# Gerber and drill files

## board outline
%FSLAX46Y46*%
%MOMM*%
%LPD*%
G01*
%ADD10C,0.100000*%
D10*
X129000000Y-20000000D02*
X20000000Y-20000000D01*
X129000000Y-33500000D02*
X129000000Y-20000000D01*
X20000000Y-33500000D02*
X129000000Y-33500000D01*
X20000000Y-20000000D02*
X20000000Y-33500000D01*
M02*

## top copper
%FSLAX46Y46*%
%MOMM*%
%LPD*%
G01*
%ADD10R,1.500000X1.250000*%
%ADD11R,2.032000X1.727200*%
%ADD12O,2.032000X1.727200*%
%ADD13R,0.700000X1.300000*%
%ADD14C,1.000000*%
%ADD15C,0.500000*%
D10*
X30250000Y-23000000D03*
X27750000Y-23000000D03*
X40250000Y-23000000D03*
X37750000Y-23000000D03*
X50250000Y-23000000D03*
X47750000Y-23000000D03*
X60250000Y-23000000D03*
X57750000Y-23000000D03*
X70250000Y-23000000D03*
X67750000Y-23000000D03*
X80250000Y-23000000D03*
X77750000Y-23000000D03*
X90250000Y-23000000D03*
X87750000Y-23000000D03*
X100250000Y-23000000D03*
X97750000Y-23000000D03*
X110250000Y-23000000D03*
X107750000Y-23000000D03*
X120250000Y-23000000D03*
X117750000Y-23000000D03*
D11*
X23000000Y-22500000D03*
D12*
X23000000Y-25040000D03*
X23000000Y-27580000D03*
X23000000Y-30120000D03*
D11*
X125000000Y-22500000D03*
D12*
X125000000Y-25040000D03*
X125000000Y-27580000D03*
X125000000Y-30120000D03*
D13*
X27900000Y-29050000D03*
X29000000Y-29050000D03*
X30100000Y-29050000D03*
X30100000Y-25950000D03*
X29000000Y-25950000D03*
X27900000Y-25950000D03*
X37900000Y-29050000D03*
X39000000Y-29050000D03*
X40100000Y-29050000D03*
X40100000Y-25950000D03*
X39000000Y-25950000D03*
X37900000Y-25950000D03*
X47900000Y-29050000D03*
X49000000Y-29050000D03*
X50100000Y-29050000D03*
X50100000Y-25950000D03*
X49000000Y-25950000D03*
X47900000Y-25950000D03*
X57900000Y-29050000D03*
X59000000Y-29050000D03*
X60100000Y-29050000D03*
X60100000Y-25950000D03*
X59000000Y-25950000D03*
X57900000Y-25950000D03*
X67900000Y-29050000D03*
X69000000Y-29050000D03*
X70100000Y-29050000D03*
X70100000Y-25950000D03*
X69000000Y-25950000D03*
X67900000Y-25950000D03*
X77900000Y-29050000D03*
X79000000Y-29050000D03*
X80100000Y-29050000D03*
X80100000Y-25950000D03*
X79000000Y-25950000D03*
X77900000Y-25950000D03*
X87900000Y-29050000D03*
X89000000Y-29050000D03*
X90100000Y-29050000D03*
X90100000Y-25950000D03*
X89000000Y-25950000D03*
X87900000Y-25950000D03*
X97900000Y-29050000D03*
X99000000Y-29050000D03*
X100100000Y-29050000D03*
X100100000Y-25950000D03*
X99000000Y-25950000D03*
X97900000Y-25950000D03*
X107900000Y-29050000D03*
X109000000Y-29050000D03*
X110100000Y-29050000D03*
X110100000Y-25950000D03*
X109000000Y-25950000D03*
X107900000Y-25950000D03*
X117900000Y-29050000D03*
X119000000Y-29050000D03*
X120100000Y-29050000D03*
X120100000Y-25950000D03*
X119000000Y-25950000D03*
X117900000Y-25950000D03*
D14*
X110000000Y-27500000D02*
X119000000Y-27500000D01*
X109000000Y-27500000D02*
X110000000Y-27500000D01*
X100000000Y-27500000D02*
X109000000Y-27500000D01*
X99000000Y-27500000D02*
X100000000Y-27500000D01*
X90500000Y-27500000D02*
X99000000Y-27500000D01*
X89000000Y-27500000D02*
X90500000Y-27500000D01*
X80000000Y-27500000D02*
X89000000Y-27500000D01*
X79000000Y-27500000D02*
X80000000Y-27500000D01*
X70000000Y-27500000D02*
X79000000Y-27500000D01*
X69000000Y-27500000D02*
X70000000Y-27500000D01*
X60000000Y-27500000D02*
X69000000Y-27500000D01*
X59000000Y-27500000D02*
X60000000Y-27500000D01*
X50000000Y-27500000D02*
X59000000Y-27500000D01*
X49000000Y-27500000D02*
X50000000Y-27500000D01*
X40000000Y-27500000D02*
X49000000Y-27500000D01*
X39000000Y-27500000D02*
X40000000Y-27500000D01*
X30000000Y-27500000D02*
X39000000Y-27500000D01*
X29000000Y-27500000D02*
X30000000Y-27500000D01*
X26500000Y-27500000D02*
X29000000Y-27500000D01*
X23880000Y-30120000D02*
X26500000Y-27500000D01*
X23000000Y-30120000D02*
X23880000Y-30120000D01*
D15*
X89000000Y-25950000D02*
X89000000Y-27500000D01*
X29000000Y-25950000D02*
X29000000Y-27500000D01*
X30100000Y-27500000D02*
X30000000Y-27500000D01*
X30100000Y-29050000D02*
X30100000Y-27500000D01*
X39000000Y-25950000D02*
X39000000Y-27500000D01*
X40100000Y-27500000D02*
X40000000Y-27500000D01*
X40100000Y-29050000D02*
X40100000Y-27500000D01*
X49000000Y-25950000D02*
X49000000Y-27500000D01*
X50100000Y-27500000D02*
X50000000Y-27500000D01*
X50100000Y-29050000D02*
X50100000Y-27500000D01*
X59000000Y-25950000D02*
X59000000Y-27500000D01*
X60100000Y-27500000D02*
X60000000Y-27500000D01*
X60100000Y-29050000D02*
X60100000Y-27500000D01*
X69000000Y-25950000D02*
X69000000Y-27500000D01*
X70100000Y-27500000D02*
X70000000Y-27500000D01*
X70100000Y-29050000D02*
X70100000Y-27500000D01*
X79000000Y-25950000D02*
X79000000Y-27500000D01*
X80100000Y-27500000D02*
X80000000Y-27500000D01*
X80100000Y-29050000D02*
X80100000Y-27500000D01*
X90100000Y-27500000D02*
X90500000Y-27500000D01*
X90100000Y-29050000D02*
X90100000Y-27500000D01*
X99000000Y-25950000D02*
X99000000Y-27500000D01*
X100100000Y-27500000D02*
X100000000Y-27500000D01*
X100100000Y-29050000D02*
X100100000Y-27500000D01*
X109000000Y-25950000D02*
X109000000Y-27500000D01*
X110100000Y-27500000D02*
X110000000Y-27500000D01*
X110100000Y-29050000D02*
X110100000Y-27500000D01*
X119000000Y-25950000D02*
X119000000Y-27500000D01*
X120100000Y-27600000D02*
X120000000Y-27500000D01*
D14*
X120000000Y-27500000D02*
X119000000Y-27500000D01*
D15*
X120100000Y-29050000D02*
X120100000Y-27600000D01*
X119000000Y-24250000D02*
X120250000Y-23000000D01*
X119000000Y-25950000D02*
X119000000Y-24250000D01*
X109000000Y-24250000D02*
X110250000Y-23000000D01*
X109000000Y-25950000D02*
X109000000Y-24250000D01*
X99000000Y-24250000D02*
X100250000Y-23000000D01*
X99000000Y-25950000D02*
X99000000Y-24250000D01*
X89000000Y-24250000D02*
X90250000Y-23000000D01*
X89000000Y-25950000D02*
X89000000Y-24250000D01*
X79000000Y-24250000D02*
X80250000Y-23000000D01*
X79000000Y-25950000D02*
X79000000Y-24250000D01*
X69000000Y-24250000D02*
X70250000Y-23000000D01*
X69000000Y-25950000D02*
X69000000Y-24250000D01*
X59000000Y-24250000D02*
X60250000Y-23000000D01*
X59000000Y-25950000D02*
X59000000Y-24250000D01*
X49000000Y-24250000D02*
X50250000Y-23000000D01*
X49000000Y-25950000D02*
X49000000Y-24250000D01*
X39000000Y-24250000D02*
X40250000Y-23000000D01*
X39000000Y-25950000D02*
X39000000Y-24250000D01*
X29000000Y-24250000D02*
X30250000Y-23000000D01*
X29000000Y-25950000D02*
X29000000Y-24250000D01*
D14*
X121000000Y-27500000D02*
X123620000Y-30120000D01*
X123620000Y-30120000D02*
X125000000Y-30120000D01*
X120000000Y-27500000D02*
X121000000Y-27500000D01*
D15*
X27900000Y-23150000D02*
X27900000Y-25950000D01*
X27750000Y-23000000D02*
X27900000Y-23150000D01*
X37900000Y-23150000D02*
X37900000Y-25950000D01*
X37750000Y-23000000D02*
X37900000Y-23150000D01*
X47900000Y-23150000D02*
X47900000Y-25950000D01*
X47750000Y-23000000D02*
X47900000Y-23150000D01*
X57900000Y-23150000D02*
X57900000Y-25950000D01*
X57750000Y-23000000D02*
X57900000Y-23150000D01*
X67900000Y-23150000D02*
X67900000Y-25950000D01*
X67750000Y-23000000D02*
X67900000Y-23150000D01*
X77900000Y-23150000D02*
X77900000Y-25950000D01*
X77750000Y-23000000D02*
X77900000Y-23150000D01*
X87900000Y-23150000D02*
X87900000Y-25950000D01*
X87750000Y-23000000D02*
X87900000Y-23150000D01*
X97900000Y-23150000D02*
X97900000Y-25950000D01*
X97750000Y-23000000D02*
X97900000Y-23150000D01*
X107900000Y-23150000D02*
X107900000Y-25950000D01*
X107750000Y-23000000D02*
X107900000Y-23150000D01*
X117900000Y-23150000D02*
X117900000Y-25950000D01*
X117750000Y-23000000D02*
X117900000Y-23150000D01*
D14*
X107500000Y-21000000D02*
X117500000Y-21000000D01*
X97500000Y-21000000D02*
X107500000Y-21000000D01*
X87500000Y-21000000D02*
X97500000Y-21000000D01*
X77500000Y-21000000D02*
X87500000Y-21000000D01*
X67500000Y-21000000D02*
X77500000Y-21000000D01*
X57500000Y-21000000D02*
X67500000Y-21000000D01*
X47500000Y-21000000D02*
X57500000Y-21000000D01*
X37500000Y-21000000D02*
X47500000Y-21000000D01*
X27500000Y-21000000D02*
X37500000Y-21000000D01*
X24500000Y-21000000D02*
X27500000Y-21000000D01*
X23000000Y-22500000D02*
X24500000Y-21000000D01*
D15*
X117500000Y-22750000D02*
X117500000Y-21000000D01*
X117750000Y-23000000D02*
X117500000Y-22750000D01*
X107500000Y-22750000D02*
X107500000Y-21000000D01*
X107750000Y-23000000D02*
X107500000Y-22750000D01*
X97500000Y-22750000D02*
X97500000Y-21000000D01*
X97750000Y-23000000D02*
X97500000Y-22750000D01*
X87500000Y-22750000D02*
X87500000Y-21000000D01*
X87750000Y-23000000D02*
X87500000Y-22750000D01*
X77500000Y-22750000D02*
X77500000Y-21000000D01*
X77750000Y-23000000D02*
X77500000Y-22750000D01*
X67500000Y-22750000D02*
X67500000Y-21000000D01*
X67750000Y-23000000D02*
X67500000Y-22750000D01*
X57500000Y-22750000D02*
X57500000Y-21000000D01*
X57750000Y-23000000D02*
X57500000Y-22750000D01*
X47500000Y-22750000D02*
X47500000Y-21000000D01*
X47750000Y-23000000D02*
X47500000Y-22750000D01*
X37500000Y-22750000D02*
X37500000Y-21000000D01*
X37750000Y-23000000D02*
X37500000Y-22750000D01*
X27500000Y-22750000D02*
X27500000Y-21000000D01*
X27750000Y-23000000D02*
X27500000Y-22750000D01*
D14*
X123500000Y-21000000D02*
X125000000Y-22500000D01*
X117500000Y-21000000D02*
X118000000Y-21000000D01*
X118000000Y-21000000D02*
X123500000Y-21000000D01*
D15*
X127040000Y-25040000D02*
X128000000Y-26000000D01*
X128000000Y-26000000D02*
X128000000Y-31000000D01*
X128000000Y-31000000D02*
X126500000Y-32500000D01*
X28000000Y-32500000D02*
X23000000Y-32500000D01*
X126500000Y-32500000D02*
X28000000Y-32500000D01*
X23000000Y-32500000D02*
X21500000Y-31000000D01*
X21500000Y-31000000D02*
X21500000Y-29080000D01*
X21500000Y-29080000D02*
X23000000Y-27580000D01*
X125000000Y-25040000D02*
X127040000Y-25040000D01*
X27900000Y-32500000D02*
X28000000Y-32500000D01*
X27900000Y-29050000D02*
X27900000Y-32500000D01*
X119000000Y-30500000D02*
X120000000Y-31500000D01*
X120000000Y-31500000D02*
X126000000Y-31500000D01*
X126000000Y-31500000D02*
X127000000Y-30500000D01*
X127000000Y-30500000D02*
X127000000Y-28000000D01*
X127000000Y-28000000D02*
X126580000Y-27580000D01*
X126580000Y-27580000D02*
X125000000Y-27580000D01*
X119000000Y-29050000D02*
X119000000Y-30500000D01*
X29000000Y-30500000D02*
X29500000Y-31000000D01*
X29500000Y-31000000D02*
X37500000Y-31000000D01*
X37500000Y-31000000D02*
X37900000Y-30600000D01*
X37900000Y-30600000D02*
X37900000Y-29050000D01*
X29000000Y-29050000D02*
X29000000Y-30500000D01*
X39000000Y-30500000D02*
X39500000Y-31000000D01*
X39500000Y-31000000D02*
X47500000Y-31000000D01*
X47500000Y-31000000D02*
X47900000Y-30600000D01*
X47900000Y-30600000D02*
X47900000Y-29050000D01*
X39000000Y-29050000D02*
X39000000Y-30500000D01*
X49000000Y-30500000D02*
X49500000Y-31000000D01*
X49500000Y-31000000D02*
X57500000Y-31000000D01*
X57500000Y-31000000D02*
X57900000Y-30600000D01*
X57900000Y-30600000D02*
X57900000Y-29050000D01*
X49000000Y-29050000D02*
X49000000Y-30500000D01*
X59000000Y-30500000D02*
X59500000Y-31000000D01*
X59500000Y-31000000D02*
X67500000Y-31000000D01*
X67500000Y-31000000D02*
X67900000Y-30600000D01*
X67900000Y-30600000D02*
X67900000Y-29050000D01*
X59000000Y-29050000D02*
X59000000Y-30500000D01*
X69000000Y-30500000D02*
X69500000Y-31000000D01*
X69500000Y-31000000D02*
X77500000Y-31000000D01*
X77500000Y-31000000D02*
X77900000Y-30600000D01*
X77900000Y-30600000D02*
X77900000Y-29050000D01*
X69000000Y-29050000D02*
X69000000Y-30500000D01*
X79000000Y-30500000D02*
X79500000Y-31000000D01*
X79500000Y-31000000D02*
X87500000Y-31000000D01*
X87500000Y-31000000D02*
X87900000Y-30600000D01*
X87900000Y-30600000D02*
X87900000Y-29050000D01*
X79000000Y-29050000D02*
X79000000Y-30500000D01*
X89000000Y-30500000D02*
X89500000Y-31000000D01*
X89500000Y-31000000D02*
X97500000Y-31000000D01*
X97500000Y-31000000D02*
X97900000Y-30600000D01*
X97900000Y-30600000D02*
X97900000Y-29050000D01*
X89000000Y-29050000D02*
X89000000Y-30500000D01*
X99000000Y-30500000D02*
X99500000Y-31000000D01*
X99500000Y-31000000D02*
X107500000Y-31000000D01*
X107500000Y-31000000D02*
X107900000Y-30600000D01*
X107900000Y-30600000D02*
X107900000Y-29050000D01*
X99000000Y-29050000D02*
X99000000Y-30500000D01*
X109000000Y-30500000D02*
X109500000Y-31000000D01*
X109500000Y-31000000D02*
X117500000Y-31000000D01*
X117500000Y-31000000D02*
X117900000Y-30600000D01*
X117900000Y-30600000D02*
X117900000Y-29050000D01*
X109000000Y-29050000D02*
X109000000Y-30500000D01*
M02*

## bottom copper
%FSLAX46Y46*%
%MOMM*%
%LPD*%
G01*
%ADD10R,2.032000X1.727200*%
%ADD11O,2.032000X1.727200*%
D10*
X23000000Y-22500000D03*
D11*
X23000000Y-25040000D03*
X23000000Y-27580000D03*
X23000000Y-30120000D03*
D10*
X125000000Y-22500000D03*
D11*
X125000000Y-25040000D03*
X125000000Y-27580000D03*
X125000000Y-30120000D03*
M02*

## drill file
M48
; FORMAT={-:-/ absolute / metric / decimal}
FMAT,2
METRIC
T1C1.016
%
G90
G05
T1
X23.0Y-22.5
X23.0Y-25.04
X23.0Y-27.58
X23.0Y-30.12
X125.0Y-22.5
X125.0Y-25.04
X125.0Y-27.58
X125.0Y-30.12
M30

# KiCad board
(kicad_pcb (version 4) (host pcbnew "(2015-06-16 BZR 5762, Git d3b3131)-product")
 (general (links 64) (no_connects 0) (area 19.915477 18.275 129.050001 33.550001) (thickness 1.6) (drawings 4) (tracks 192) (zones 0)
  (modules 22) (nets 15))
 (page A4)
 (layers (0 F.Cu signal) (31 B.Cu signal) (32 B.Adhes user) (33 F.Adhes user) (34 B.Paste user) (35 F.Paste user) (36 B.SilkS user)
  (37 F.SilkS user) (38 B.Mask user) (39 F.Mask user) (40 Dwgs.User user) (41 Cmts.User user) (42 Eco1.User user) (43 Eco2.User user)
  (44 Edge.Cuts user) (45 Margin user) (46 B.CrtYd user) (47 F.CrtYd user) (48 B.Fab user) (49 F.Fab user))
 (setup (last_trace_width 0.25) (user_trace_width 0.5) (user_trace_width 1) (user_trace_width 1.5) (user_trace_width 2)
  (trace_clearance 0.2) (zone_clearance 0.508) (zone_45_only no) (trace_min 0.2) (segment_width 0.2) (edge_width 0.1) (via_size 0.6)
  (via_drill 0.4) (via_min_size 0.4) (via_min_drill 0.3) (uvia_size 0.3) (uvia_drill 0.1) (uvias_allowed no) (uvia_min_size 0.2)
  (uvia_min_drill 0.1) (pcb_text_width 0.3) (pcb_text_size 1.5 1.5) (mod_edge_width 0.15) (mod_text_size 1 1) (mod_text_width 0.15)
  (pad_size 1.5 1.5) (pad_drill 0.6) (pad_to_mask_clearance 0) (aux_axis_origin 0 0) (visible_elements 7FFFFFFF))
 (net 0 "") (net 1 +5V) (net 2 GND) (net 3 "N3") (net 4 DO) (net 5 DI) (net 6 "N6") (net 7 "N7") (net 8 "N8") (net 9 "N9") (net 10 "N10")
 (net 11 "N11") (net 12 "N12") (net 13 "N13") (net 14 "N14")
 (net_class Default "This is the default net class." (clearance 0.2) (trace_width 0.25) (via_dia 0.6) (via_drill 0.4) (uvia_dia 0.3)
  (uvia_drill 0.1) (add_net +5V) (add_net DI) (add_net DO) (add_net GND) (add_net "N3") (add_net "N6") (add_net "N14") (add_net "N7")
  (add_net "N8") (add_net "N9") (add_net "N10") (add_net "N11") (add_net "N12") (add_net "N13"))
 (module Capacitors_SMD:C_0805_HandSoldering (layer F.Cu) (at 29 23 180)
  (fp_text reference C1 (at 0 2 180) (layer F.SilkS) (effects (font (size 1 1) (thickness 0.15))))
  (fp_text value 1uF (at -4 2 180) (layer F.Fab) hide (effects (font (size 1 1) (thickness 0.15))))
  (pad 1 smd rect (at -1.25 0 180) (size 1.5 1.25) (layers F.Cu F.Paste F.Mask) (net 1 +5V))
  (pad 2 smd rect (at 1.25 0 180) (size 1.5 1.25) (layers F.Cu F.Paste F.Mask) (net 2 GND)))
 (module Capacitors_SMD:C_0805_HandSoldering (layer F.Cu) (at 39 23 180)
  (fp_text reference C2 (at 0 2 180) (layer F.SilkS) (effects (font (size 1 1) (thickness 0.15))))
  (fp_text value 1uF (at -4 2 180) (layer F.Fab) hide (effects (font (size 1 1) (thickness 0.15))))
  (pad 1 smd rect (at -1.25 0 180) (size 1.5 1.25) (layers F.Cu F.Paste F.Mask) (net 1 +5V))
  (pad 2 smd rect (at 1.25 0 180) (size 1.5 1.25) (layers F.Cu F.Paste F.Mask) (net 2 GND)))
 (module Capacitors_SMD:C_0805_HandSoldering (layer F.Cu) (at 49 23 180)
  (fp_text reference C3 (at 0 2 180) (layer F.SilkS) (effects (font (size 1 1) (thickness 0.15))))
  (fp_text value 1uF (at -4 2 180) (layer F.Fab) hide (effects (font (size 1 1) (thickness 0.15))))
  (pad 1 smd rect (at -1.25 0 180) (size 1.5 1.25) (layers F.Cu F.Paste F.Mask) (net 1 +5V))
  (pad 2 smd rect (at 1.25 0 180) (size 1.5 1.25) (layers F.Cu F.Paste F.Mask) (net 2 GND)))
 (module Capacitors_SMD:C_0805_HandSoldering (layer F.Cu) (at 59 23 180)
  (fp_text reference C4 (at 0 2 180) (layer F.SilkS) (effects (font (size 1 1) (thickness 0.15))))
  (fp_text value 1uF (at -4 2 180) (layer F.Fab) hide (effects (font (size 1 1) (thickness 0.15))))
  (pad 1 smd rect (at -1.25 0 180) (size 1.5 1.25) (layers F.Cu F.Paste F.Mask) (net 1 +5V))
  (pad 2 smd rect (at 1.25 0 180) (size 1.5 1.25) (layers F.Cu F.Paste F.Mask) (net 2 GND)))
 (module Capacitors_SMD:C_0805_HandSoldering (layer F.Cu) (at 69 23 180)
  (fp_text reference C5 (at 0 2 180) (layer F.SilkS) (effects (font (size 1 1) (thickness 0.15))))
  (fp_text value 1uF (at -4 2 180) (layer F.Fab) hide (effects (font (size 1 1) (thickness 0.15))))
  (pad 1 smd rect (at -1.25 0 180) (size 1.5 1.25) (layers F.Cu F.Paste F.Mask) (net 1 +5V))
  (pad 2 smd rect (at 1.25 0 180) (size 1.5 1.25) (layers F.Cu F.Paste F.Mask) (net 2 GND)))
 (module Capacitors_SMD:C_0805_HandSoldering (layer F.Cu) (at 79 23 180)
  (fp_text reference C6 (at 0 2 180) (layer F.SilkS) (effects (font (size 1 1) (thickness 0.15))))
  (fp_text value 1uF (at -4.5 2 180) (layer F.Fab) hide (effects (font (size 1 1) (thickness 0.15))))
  (pad 1 smd rect (at -1.25 0 180) (size 1.5 1.25) (layers F.Cu F.Paste F.Mask) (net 1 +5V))
  (pad 2 smd rect (at 1.25 0 180) (size 1.5 1.25) (layers F.Cu F.Paste F.Mask) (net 2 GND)))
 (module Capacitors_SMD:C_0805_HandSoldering (layer F.Cu) (at 89 23 180)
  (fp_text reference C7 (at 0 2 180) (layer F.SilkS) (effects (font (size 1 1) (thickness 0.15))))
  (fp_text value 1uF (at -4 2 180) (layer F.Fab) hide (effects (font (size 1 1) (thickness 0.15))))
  (pad 1 smd rect (at -1.25 0 180) (size 1.5 1.25) (layers F.Cu F.Paste F.Mask) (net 1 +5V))
  (pad 2 smd rect (at 1.25 0 180) (size 1.5 1.25) (layers F.Cu F.Paste F.Mask) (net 2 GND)))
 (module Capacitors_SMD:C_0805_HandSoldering (layer F.Cu) (at 99 23 180)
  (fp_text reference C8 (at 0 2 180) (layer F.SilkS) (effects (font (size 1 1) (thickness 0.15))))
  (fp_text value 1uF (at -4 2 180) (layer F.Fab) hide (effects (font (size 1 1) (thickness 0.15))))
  (pad 1 smd rect (at -1.25 0 180) (size 1.5 1.25) (layers F.Cu F.Paste F.Mask) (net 1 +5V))
  (pad 2 smd rect (at 1.25 0 180) (size 1.5 1.25) (layers F.Cu F.Paste F.Mask) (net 2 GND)))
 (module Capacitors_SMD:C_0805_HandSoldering (layer F.Cu) (at 109 23 180)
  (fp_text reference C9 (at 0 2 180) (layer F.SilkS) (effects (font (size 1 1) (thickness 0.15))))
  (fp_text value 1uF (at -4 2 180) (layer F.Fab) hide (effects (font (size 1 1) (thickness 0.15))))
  (pad 1 smd rect (at -1.25 0 180) (size 1.5 1.25) (layers F.Cu F.Paste F.Mask) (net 1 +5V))
  (pad 2 smd rect (at 1.25 0 180) (size 1.5 1.25) (layers F.Cu F.Paste F.Mask) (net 2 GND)))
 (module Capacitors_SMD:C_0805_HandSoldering (layer F.Cu) (at 119 23 180)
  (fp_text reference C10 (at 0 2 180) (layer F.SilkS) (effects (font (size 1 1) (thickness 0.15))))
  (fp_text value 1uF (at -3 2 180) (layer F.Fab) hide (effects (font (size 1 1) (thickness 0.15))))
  (pad 1 smd rect (at -1.25 0 180) (size 1.5 1.25) (layers F.Cu F.Paste F.Mask) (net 1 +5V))
  (pad 2 smd rect (at 1.25 0 180) (size 1.5 1.25) (layers F.Cu F.Paste F.Mask) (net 2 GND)))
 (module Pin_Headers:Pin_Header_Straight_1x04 (layer F.Cu) (at 23 22.5)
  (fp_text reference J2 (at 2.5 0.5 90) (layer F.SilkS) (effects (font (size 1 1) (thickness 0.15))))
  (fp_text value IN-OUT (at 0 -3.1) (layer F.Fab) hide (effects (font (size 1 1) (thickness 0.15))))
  (pad 1 thru_hole rect (at 0 0) (size 2.032 1.7272) (drill 1.016) (layers *.Cu *.Mask F.SilkS) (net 2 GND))
  (pad 2 thru_hole oval (at 0 2.54) (size 2.032 1.7272) (drill 1.016) (layers *.Cu *.Mask F.SilkS) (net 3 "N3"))
  (pad 3 thru_hole oval (at 0 5.08) (size 2.032 1.7272) (drill 1.016) (layers *.Cu *.Mask F.SilkS) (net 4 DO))
  (pad 4 thru_hole oval (at 0 7.62) (size 2.032 1.7272) (drill 1.016) (layers *.Cu *.Mask F.SilkS) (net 1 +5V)))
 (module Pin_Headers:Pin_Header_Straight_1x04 (layer F.Cu) (at 125 22.5)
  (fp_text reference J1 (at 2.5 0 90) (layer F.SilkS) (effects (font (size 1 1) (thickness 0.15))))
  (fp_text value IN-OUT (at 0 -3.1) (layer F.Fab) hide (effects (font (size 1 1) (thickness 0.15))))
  (pad 1 thru_hole rect (at 0 0) (size 2.032 1.7272) (drill 1.016) (layers *.Cu *.Mask F.SilkS) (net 2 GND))
  (pad 2 thru_hole oval (at 0 2.54) (size 2.032 1.7272) (drill 1.016) (layers *.Cu *.Mask F.SilkS) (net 4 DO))
  (pad 3 thru_hole oval (at 0 5.08) (size 2.032 1.7272) (drill 1.016) (layers *.Cu *.Mask F.SilkS) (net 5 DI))
  (pad 4 thru_hole oval (at 0 7.62) (size 2.032 1.7272) (drill 1.016) (layers *.Cu *.Mask F.SilkS) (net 1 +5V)))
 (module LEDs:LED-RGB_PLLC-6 (layer F.Cu) (at 29 27.5 90)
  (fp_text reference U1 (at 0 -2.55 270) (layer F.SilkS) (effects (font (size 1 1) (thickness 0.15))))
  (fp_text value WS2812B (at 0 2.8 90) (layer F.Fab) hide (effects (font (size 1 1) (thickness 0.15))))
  (pad 1 smd rect (at -1.55 -1.1 180) (size 0.7 1.3) (layers F.Cu F.Paste F.Mask) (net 4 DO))
  (pad 2 smd rect (at -1.55 0 180) (size 0.7 1.3) (layers F.Cu F.Paste F.Mask) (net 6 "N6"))
  (pad 3 smd rect (at -1.55 1.1 180) (size 0.7 1.3) (layers F.Cu F.Paste F.Mask) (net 1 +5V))
  (pad 4 smd rect (at 1.55 1.1 180) (size 0.7 1.3) (layers F.Cu F.Paste F.Mask))
  (pad 5 smd rect (at 1.55 0 180) (size 0.7 1.3) (layers F.Cu F.Paste F.Mask) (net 1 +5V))
  (pad 6 smd rect (at 1.55 -1.1 180) (size 0.7 1.3) (layers F.Cu F.Paste F.Mask) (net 2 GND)))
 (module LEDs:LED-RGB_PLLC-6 (layer F.Cu) (at 39 27.5 90)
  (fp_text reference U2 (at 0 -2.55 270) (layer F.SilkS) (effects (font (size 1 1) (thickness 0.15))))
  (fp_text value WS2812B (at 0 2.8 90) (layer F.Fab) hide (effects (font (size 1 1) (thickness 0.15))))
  (pad 1 smd rect (at -1.55 -1.1 180) (size 0.7 1.3) (layers F.Cu F.Paste F.Mask) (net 6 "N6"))
  (pad 2 smd rect (at -1.55 0 180) (size 0.7 1.3) (layers F.Cu F.Paste F.Mask) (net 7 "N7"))
  (pad 3 smd rect (at -1.55 1.1 180) (size 0.7 1.3) (layers F.Cu F.Paste F.Mask) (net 1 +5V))
  (pad 4 smd rect (at 1.55 1.1 180) (size 0.7 1.3) (layers F.Cu F.Paste F.Mask))
  (pad 5 smd rect (at 1.55 0 180) (size 0.7 1.3) (layers F.Cu F.Paste F.Mask) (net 1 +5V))
  (pad 6 smd rect (at 1.55 -1.1 180) (size 0.7 1.3) (layers F.Cu F.Paste F.Mask) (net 2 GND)))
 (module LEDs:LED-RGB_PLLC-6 (layer F.Cu) (at 49 27.5 90)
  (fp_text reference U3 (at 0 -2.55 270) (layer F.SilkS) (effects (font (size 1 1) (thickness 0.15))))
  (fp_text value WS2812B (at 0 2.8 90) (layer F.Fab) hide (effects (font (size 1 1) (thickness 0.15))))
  (pad 1 smd rect (at -1.55 -1.1 180) (size 0.7 1.3) (layers F.Cu F.Paste F.Mask) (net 7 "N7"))
  (pad 2 smd rect (at -1.55 0 180) (size 0.7 1.3) (layers F.Cu F.Paste F.Mask) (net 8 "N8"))
  (pad 3 smd rect (at -1.55 1.1 180) (size 0.7 1.3) (layers F.Cu F.Paste F.Mask) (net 1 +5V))
  (pad 4 smd rect (at 1.55 1.1 180) (size 0.7 1.3) (layers F.Cu F.Paste F.Mask))
  (pad 5 smd rect (at 1.55 0 180) (size 0.7 1.3) (layers F.Cu F.Paste F.Mask) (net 1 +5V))
  (pad 6 smd rect (at 1.55 -1.1 180) (size 0.7 1.3) (layers F.Cu F.Paste F.Mask) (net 2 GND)))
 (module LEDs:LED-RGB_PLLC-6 (layer F.Cu) (at 59 27.5 90)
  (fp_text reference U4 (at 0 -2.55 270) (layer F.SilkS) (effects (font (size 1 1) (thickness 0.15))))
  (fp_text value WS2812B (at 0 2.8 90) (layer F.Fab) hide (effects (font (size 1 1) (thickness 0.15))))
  (pad 1 smd rect (at -1.55 -1.1 180) (size 0.7 1.3) (layers F.Cu F.Paste F.Mask) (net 8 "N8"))
  (pad 2 smd rect (at -1.55 0 180) (size 0.7 1.3) (layers F.Cu F.Paste F.Mask) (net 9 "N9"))
  (pad 3 smd rect (at -1.55 1.1 180) (size 0.7 1.3) (layers F.Cu F.Paste F.Mask) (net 1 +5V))
  (pad 4 smd rect (at 1.55 1.1 180) (size 0.7 1.3) (layers F.Cu F.Paste F.Mask))
  (pad 5 smd rect (at 1.55 0 180) (size 0.7 1.3) (layers F.Cu F.Paste F.Mask) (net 1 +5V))
  (pad 6 smd rect (at 1.55 -1.1 180) (size 0.7 1.3) (layers F.Cu F.Paste F.Mask) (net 2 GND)))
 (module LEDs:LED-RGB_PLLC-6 (layer F.Cu) (at 69 27.5 90)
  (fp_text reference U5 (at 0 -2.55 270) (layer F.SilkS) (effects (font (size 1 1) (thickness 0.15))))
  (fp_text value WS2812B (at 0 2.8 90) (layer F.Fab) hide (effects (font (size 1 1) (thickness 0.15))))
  (pad 1 smd rect (at -1.55 -1.1 180) (size 0.7 1.3) (layers F.Cu F.Paste F.Mask) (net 9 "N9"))
  (pad 2 smd rect (at -1.55 0 180) (size 0.7 1.3) (layers F.Cu F.Paste F.Mask) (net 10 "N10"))
  (pad 3 smd rect (at -1.55 1.1 180) (size 0.7 1.3) (layers F.Cu F.Paste F.Mask) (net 1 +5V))
  (pad 4 smd rect (at 1.55 1.1 180) (size 0.7 1.3) (layers F.Cu F.Paste F.Mask))
  (pad 5 smd rect (at 1.55 0 180) (size 0.7 1.3) (layers F.Cu F.Paste F.Mask) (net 1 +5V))
  (pad 6 smd rect (at 1.55 -1.1 180) (size 0.7 1.3) (layers F.Cu F.Paste F.Mask) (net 2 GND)))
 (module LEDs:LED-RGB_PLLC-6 (layer F.Cu) (at 79 27.5 90)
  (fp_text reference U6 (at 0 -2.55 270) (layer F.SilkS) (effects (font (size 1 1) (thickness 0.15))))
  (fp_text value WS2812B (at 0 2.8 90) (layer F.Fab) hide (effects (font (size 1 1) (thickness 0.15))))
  (pad 1 smd rect (at -1.55 -1.1 180) (size 0.7 1.3) (layers F.Cu F.Paste F.Mask) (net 10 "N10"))
  (pad 2 smd rect (at -1.55 0 180) (size 0.7 1.3) (layers F.Cu F.Paste F.Mask) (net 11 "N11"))
  (pad 3 smd rect (at -1.55 1.1 180) (size 0.7 1.3) (layers F.Cu F.Paste F.Mask) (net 1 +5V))
  (pad 4 smd rect (at 1.55 1.1 180) (size 0.7 1.3) (layers F.Cu F.Paste F.Mask))
  (pad 5 smd rect (at 1.55 0 180) (size 0.7 1.3) (layers F.Cu F.Paste F.Mask) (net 1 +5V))
  (pad 6 smd rect (at 1.55 -1.1 180) (size 0.7 1.3) (layers F.Cu F.Paste F.Mask) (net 2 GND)))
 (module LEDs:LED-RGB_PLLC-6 (layer F.Cu) (at 89 27.5 90)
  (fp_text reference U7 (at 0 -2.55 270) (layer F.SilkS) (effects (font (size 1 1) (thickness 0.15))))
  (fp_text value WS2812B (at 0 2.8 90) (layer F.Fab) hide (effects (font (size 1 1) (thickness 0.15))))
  (pad 1 smd rect (at -1.55 -1.1 180) (size 0.7 1.3) (layers F.Cu F.Paste F.Mask) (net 11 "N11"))
  (pad 2 smd rect (at -1.55 0 180) (size 0.7 1.3) (layers F.Cu F.Paste F.Mask) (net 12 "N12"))
  (pad 3 smd rect (at -1.55 1.1 180) (size 0.7 1.3) (layers F.Cu F.Paste F.Mask) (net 1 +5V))
  (pad 4 smd rect (at 1.55 1.1 180) (size 0.7 1.3) (layers F.Cu F.Paste F.Mask))
  (pad 5 smd rect (at 1.55 0 180) (size 0.7 1.3) (layers F.Cu F.Paste F.Mask) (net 1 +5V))
  (pad 6 smd rect (at 1.55 -1.1 180) (size 0.7 1.3) (layers F.Cu F.Paste F.Mask) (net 2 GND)))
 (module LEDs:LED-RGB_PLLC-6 (layer F.Cu) (at 99 27.5 90)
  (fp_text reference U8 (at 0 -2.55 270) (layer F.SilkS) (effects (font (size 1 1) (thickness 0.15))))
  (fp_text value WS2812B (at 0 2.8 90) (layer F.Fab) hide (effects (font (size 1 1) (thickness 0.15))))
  (pad 1 smd rect (at -1.55 -1.1 180) (size 0.7 1.3) (layers F.Cu F.Paste F.Mask) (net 12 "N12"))
  (pad 2 smd rect (at -1.55 0 180) (size 0.7 1.3) (layers F.Cu F.Paste F.Mask) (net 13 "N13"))
  (pad 3 smd rect (at -1.55 1.1 180) (size 0.7 1.3) (layers F.Cu F.Paste F.Mask) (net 1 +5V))
  (pad 4 smd rect (at 1.55 1.1 180) (size 0.7 1.3) (layers F.Cu F.Paste F.Mask))
  (pad 5 smd rect (at 1.55 0 180) (size 0.7 1.3) (layers F.Cu F.Paste F.Mask) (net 1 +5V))
  (pad 6 smd rect (at 1.55 -1.1 180) (size 0.7 1.3) (layers F.Cu F.Paste F.Mask) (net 2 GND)))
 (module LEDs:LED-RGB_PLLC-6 (layer F.Cu) (at 109 27.5 90)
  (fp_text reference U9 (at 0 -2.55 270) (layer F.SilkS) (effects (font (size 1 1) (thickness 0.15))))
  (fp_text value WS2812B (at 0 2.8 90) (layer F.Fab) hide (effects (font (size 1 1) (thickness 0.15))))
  (pad 1 smd rect (at -1.55 -1.1 180) (size 0.7 1.3) (layers F.Cu F.Paste F.Mask) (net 13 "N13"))
  (pad 2 smd rect (at -1.55 0 180) (size 0.7 1.3) (layers F.Cu F.Paste F.Mask) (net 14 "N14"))
  (pad 3 smd rect (at -1.55 1.1 180) (size 0.7 1.3) (layers F.Cu F.Paste F.Mask) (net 1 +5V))
  (pad 4 smd rect (at 1.55 1.1 180) (size 0.7 1.3) (layers F.Cu F.Paste F.Mask))
  (pad 5 smd rect (at 1.55 0 180) (size 0.7 1.3) (layers F.Cu F.Paste F.Mask) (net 1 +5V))
  (pad 6 smd rect (at 1.55 -1.1 180) (size 0.7 1.3) (layers F.Cu F.Paste F.Mask) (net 2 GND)))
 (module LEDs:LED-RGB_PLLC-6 (layer F.Cu) (at 119 27.5 90)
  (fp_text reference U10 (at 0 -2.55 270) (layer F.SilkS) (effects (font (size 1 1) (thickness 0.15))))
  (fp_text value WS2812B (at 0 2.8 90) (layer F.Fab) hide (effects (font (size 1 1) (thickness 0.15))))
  (pad 1 smd rect (at -1.55 -1.1 180) (size 0.7 1.3) (layers F.Cu F.Paste F.Mask) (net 14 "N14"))
  (pad 2 smd rect (at -1.55 0 180) (size 0.7 1.3) (layers F.Cu F.Paste F.Mask) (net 5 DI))
  (pad 3 smd rect (at -1.55 1.1 180) (size 0.7 1.3) (layers F.Cu F.Paste F.Mask) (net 1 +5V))
  (pad 4 smd rect (at 1.55 1.1 180) (size 0.7 1.3) (layers F.Cu F.Paste F.Mask))
  (pad 5 smd rect (at 1.55 0 180) (size 0.7 1.3) (layers F.Cu F.Paste F.Mask) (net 1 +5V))
  (pad 6 smd rect (at 1.55 -1.1 180) (size 0.7 1.3) (layers F.Cu F.Paste F.Mask) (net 2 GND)))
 (gr_line (start 129 20) (end 20 20) (angle 90) (layer Edge.Cuts) (width 0.1))
 (gr_line (start 129 33.5) (end 129 20) (angle 90) (layer Edge.Cuts) (width 0.1))
 (gr_line (start 20 33.5) (end 129 33.5) (angle 90) (layer Edge.Cuts) (width 0.1))
 (gr_line (start 20 20) (end 20 33.5) (angle 90) (layer Edge.Cuts) (width 0.1))
 (segment (start 110 27.5) (end 119 27.5) (width 1) (layer F.Cu) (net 1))
 (segment (start 109 27.5) (end 110 27.5) (width 1) (layer F.Cu) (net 1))
 (segment (start 100 27.5) (end 109 27.5) (width 1) (layer F.Cu) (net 1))
 (segment (start 99 27.5) (end 100 27.5) (width 1) (layer F.Cu) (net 1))
 (segment (start 90.5 27.5) (end 99 27.5) (width 1) (layer F.Cu) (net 1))
 (segment (start 89 27.5) (end 90.5 27.5) (width 1) (layer F.Cu) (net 1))
 (segment (start 80 27.5) (end 89 27.5) (width 1) (layer F.Cu) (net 1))
 (segment (start 79 27.5) (end 80 27.5) (width 1) (layer F.Cu) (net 1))
 (segment (start 70 27.5) (end 79 27.5) (width 1) (layer F.Cu) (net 1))
 (segment (start 69 27.5) (end 70 27.5) (width 1) (layer F.Cu) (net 1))
 (segment (start 60 27.5) (end 69 27.5) (width 1) (layer F.Cu) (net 1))
 (segment (start 59 27.5) (end 60 27.5) (width 1) (layer F.Cu) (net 1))
 (segment (start 50 27.5) (end 59 27.5) (width 1) (layer F.Cu) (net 1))
 (segment (start 49 27.5) (end 50 27.5) (width 1) (layer F.Cu) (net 1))
 (segment (start 40 27.5) (end 49 27.5) (width 1) (layer F.Cu) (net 1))
 (segment (start 39 27.5) (end 40 27.5) (width 1) (layer F.Cu) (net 1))
 (segment (start 30 27.5) (end 39 27.5) (width 1) (layer F.Cu) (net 1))
 (segment (start 29 27.5) (end 30 27.5) (width 1) (layer F.Cu) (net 1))
 (segment (start 26.5 27.5) (end 29 27.5) (width 1) (layer F.Cu) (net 1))
 (segment (start 23.88 30.12) (end 26.5 27.5) (width 1) (layer F.Cu) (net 1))
 (segment (start 23 30.12) (end 23.88 30.12) (width 1) (layer F.Cu) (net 1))
 (segment (start 89 25.95) (end 89 27.5) (width 0.5) (layer F.Cu) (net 1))
 (segment (start 29 25.95) (end 29 27.5) (width 0.5) (layer F.Cu) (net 1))
 (segment (start 30.1 27.5) (end 30 27.5) (width 0.5) (layer F.Cu) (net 1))
 (segment (start 30.1 29.05) (end 30.1 27.5) (width 0.5) (layer F.Cu) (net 1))
 (segment (start 39 25.95) (end 39 27.5) (width 0.5) (layer F.Cu) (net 1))
 (segment (start 40.1 27.5) (end 40 27.5) (width 0.5) (layer F.Cu) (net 1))
 (segment (start 40.1 29.05) (end 40.1 27.5) (width 0.5) (layer F.Cu) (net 1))
 (segment (start 49 25.95) (end 49 27.5) (width 0.5) (layer F.Cu) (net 1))
 (segment (start 50.1 27.5) (end 50 27.5) (width 0.5) (layer F.Cu) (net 1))
 (segment (start 50.1 29.05) (end 50.1 27.5) (width 0.5) (layer F.Cu) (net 1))
 (segment (start 59 25.95) (end 59 27.5) (width 0.5) (layer F.Cu) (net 1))
 (segment (start 60.1 27.5) (end 60 27.5) (width 0.5) (layer F.Cu) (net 1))
 (segment (start 60.1 29.05) (end 60.1 27.5) (width 0.5) (layer F.Cu) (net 1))
 (segment (start 69 25.95) (end 69 27.5) (width 0.5) (layer F.Cu) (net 1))
 (segment (start 70.1 27.5) (end 70 27.5) (width 0.5) (layer F.Cu) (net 1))
 (segment (start 70.1 29.05) (end 70.1 27.5) (width 0.5) (layer F.Cu) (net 1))
 (segment (start 79 25.95) (end 79 27.5) (width 0.5) (layer F.Cu) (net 1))
 (segment (start 80.1 27.5) (end 80 27.5) (width 0.5) (layer F.Cu) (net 1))
 (segment (start 80.1 29.05) (end 80.1 27.5) (width 0.5) (layer F.Cu) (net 1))
 (segment (start 90.1 27.5) (end 90.5 27.5) (width 0.5) (layer F.Cu) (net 1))
 (segment (start 90.1 29.05) (end 90.1 27.5) (width 0.5) (layer F.Cu) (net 1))
 (segment (start 99 25.95) (end 99 27.5) (width 0.5) (layer F.Cu) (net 1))
 (segment (start 100.1 27.5) (end 100 27.5) (width 0.5) (layer F.Cu) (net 1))
 (segment (start 100.1 29.05) (end 100.1 27.5) (width 0.5) (layer F.Cu) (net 1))
 (segment (start 109 25.95) (end 109 27.5) (width 0.5) (layer F.Cu) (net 1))
 (segment (start 110.1 27.5) (end 110 27.5) (width 0.5) (layer F.Cu) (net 1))
 (segment (start 110.1 29.05) (end 110.1 27.5) (width 0.5) (layer F.Cu) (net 1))
 (segment (start 119 25.95) (end 119 27.5) (width 0.5) (layer F.Cu) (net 1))
 (segment (start 120.1 27.6) (end 120 27.5) (width 0.5) (layer F.Cu) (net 1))
 (segment (start 120 27.5) (end 119 27.5) (width 1) (layer F.Cu) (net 1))
 (segment (start 120.1 29.05) (end 120.1 27.6) (width 0.5) (layer F.Cu) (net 1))
 (segment (start 119 24.25) (end 120.25 23) (width 0.5) (layer F.Cu) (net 1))
 (segment (start 119 25.95) (end 119 24.25) (width 0.5) (layer F.Cu) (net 1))
 (segment (start 109 24.25) (end 110.25 23) (width 0.5) (layer F.Cu) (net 1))
 (segment (start 109 25.95) (end 109 24.25) (width 0.5) (layer F.Cu) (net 1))
 (segment (start 99 24.25) (end 100.25 23) (width 0.5) (layer F.Cu) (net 1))
 (segment (start 99 25.95) (end 99 24.25) (width 0.5) (layer F.Cu) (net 1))
 (segment (start 89 24.25) (end 90.25 23) (width 0.5) (layer F.Cu) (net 1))
 (segment (start 89 25.95) (end 89 24.25) (width 0.5) (layer F.Cu) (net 1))
 (segment (start 79 24.25) (end 80.25 23) (width 0.5) (layer F.Cu) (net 1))
 (segment (start 79 25.95) (end 79 24.25) (width 0.5) (layer F.Cu) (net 1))
 (segment (start 69 24.25) (end 70.25 23) (width 0.5) (layer F.Cu) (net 1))
 (segment (start 69 25.95) (end 69 24.25) (width 0.5) (layer F.Cu) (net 1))
 (segment (start 59 24.25) (end 60.25 23) (width 0.5) (layer F.Cu) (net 1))
 (segment (start 59 25.95) (end 59 24.25) (width 0.5) (layer F.Cu) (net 1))
 (segment (start 49 24.25) (end 50.25 23) (width 0.5) (layer F.Cu) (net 1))
 (segment (start 49 25.95) (end 49 24.25) (width 0.5) (layer F.Cu) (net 1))
 (segment (start 39 24.25) (end 40.25 23) (width 0.5) (layer F.Cu) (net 1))
 (segment (start 39 25.95) (end 39 24.25) (width 0.5) (layer F.Cu) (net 1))
 (segment (start 29 24.25) (end 30.25 23) (width 0.5) (layer F.Cu) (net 1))
 (segment (start 29 25.95) (end 29 24.25) (width 0.5) (layer F.Cu) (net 1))
 (segment (start 121 27.5) (end 123.62 30.12) (width 1) (layer F.Cu) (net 1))
 (segment (start 123.62 30.12) (end 125 30.12) (width 1) (layer F.Cu) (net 1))
 (segment (start 120 27.5) (end 121 27.5) (width 1) (layer F.Cu) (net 1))
 (segment (start 27.9 23.15) (end 27.9 25.95) (width 0.5) (layer F.Cu) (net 2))
 (segment (start 27.75 23) (end 27.9 23.15) (width 0.5) (layer F.Cu) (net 2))
 (segment (start 37.9 23.15) (end 37.9 25.95) (width 0.5) (layer F.Cu) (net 2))
 (segment (start 37.75 23) (end 37.9 23.15) (width 0.5) (layer F.Cu) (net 2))
 (segment (start 47.9 23.15) (end 47.9 25.95) (width 0.5) (layer F.Cu) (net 2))
 (segment (start 47.75 23) (end 47.9 23.15) (width 0.5) (layer F.Cu) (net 2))
 (segment (start 57.9 23.15) (end 57.9 25.95) (width 0.5) (layer F.Cu) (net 2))
 (segment (start 57.75 23) (end 57.9 23.15) (width 0.5) (layer F.Cu) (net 2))
 (segment (start 67.9 23.15) (end 67.9 25.95) (width 0.5) (layer F.Cu) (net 2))
 (segment (start 67.75 23) (end 67.9 23.15) (width 0.5) (layer F.Cu) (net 2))
 (segment (start 77.9 23.15) (end 77.9 25.95) (width 0.5) (layer F.Cu) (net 2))
 (segment (start 77.75 23) (end 77.9 23.15) (width 0.5) (layer F.Cu) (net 2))
 (segment (start 87.9 23.15) (end 87.9 25.95) (width 0.5) (layer F.Cu) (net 2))
 (segment (start 87.75 23) (end 87.9 23.15) (width 0.5) (layer F.Cu) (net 2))
 (segment (start 97.9 23.15) (end 97.9 25.95) (width 0.5) (layer F.Cu) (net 2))
 (segment (start 97.75 23) (end 97.9 23.15) (width 0.5) (layer F.Cu) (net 2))
 (segment (start 107.9 23.15) (end 107.9 25.95) (width 0.5) (layer F.Cu) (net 2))
 (segment (start 107.75 23) (end 107.9 23.15) (width 0.5) (layer F.Cu) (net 2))
 (segment (start 117.9 23.15) (end 117.9 25.95) (width 0.5) (layer F.Cu) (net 2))
 (segment (start 117.75 23) (end 117.9 23.15) (width 0.5) (layer F.Cu) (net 2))
 (segment (start 107.5 21) (end 117.5 21) (width 1) (layer F.Cu) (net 2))
 (segment (start 97.5 21) (end 107.5 21) (width 1) (layer F.Cu) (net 2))
 (segment (start 87.5 21) (end 97.5 21) (width 1) (layer F.Cu) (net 2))
 (segment (start 77.5 21) (end 87.5 21) (width 1) (layer F.Cu) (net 2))
 (segment (start 67.5 21) (end 77.5 21) (width 1) (layer F.Cu) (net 2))
 (segment (start 57.5 21) (end 67.5 21) (width 1) (layer F.Cu) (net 2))
 (segment (start 47.5 21) (end 57.5 21) (width 1) (layer F.Cu) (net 2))
 (segment (start 37.5 21) (end 47.5 21) (width 1) (layer F.Cu) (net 2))
 (segment (start 27.5 21) (end 37.5 21) (width 1) (layer F.Cu) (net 2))
 (segment (start 24.5 21) (end 27.5 21) (width 1) (layer F.Cu) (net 2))
 (segment (start 23 22.5) (end 24.5 21) (width 1) (layer F.Cu) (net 2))
 (segment (start 117.5 22.75) (end 117.5 21) (width 0.5) (layer F.Cu) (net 2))
 (segment (start 117.75 23) (end 117.5 22.75) (width 0.5) (layer F.Cu) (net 2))
 (segment (start 107.5 22.75) (end 107.5 21) (width 0.5) (layer F.Cu) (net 2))
 (segment (start 107.75 23) (end 107.5 22.75) (width 0.5) (layer F.Cu) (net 2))
 (segment (start 97.5 22.75) (end 97.5 21) (width 0.5) (layer F.Cu) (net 2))
 (segment (start 97.75 23) (end 97.5 22.75) (width 0.5) (layer F.Cu) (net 2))
 (segment (start 87.5 22.75) (end 87.5 21) (width 0.5) (layer F.Cu) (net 2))
 (segment (start 87.75 23) (end 87.5 22.75) (width 0.5) (layer F.Cu) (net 2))
 (segment (start 77.5 22.75) (end 77.5 21) (width 0.5) (layer F.Cu) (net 2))
 (segment (start 77.75 23) (end 77.5 22.75) (width 0.5) (layer F.Cu) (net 2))
 (segment (start 67.5 22.75) (end 67.5 21) (width 0.5) (layer F.Cu) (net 2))
 (segment (start 67.75 23) (end 67.5 22.75) (width 0.5) (layer F.Cu) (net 2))
 (segment (start 57.5 22.75) (end 57.5 21) (width 0.5) (layer F.Cu) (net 2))
 (segment (start 57.75 23) (end 57.5 22.75) (width 0.5) (layer F.Cu) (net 2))
 (segment (start 47.5 22.75) (end 47.5 21) (width 0.5) (layer F.Cu) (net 2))
 (segment (start 47.75 23) (end 47.5 22.75) (width 0.5) (layer F.Cu) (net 2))
 (segment (start 37.5 22.75) (end 37.5 21) (width 0.5) (layer F.Cu) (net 2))
 (segment (start 37.75 23) (end 37.5 22.75) (width 0.5) (layer F.Cu) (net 2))
 (segment (start 27.5 22.75) (end 27.5 21) (width 0.5) (layer F.Cu) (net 2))
 (segment (start 27.75 23) (end 27.5 22.75) (width 0.5) (layer F.Cu) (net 2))
 (segment (start 123.5 21) (end 125 22.5) (width 1) (layer F.Cu) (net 2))
 (segment (start 117.5 21) (end 118 21) (width 1) (layer F.Cu) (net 2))
 (segment (start 118 21) (end 123.5 21) (width 1) (layer F.Cu) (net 2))
 (segment (start 127.04 25.04) (end 128 26) (width 0.5) (layer F.Cu) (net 4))
 (segment (start 128 26) (end 128 31) (width 0.5) (layer F.Cu) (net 4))
 (segment (start 128 31) (end 126.5 32.5) (width 0.5) (layer F.Cu) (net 4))
 (segment (start 28 32.5) (end 23 32.5) (width 0.5) (layer F.Cu) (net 4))
 (segment (start 126.5 32.5) (end 28 32.5) (width 0.5) (layer F.Cu) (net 4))
 (segment (start 23 32.5) (end 21.5 31) (width 0.5) (layer F.Cu) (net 4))
 (segment (start 21.5 31) (end 21.5 29.08) (width 0.5) (layer F.Cu) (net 4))
 (segment (start 21.5 29.08) (end 23 27.58) (width 0.5) (layer F.Cu) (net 4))
 (segment (start 125 25.04) (end 127.04 25.04) (width 0.5) (layer F.Cu) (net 4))
 (segment (start 27.9 32.5) (end 28 32.5) (width 0.5) (layer F.Cu) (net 4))
 (segment (start 27.9 29.05) (end 27.9 32.5) (width 0.5) (layer F.Cu) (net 4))
 (segment (start 119 30.5) (end 120 31.5) (width 0.5) (layer F.Cu) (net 5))
 (segment (start 120 31.5) (end 126 31.5) (width 0.5) (layer F.Cu) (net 5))
 (segment (start 126 31.5) (end 127 30.5) (width 0.5) (layer F.Cu) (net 5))
 (segment (start 127 30.5) (end 127 28) (width 0.5) (layer F.Cu) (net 5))
 (segment (start 127 28) (end 126.58 27.58) (width 0.5) (layer F.Cu) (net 5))
 (segment (start 126.58 27.58) (end 125 27.58) (width 0.5) (layer F.Cu) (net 5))
 (segment (start 119 29.05) (end 119 30.5) (width 0.5) (layer F.Cu) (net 5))
 (segment (start 29 30.5) (end 29.5 31) (width 0.5) (layer F.Cu) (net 6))
 (segment (start 29.5 31) (end 37.5 31) (width 0.5) (layer F.Cu) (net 6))
 (segment (start 37.5 31) (end 37.9 30.6) (width 0.5) (layer F.Cu) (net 6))
 (segment (start 37.9 30.6) (end 37.9 29.05) (width 0.5) (layer F.Cu) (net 6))
 (segment (start 29 29.05) (end 29 30.5) (width 0.5) (layer F.Cu) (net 6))
 (segment (start 39 30.5) (end 39.5 31) (width 0.5) (layer F.Cu) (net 7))
 (segment (start 39.5 31) (end 47.5 31) (width 0.5) (layer F.Cu) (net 7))
 (segment (start 47.5 31) (end 47.9 30.6) (width 0.5) (layer F.Cu) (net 7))
 (segment (start 47.9 30.6) (end 47.9 29.05) (width 0.5) (layer F.Cu) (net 7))
 (segment (start 39 29.05) (end 39 30.5) (width 0.5) (layer F.Cu) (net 7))
 (segment (start 49 30.5) (end 49.5 31) (width 0.5) (layer F.Cu) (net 8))
 (segment (start 49.5 31) (end 57.5 31) (width 0.5) (layer F.Cu) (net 8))
 (segment (start 57.5 31) (end 57.9 30.6) (width 0.5) (layer F.Cu) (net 8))
 (segment (start 57.9 30.6) (end 57.9 29.05) (width 0.5) (layer F.Cu) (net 8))
 (segment (start 49 29.05) (end 49 30.5) (width 0.5) (layer F.Cu) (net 8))
 (segment (start 59 30.5) (end 59.5 31) (width 0.5) (layer F.Cu) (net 9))
 (segment (start 59.5 31) (end 67.5 31) (width 0.5) (layer F.Cu) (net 9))
 (segment (start 67.5 31) (end 67.9 30.6) (width 0.5) (layer F.Cu) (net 9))
 (segment (start 67.9 30.6) (end 67.9 29.05) (width 0.5) (layer F.Cu) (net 9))
 (segment (start 59 29.05) (end 59 30.5) (width 0.5) (layer F.Cu) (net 9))
 (segment (start 69 30.5) (end 69.5 31) (width 0.5) (layer F.Cu) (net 10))
 (segment (start 69.5 31) (end 77.5 31) (width 0.5) (layer F.Cu) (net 10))
 (segment (start 77.5 31) (end 77.9 30.6) (width 0.5) (layer F.Cu) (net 10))
 (segment (start 77.9 30.6) (end 77.9 29.05) (width 0.5) (layer F.Cu) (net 10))
 (segment (start 69 29.05) (end 69 30.5) (width 0.5) (layer F.Cu) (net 10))
 (segment (start 79 30.5) (end 79.5 31) (width 0.5) (layer F.Cu) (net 11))
 (segment (start 79.5 31) (end 87.5 31) (width 0.5) (layer F.Cu) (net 11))
 (segment (start 87.5 31) (end 87.9 30.6) (width 0.5) (layer F.Cu) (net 11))
 (segment (start 87.9 30.6) (end 87.9 29.05) (width 0.5) (layer F.Cu) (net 11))
 (segment (start 79 29.05) (end 79 30.5) (width 0.5) (layer F.Cu) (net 11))
 (segment (start 89 30.5) (end 89.5 31) (width 0.5) (layer F.Cu) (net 12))
 (segment (start 89.5 31) (end 97.5 31) (width 0.5) (layer F.Cu) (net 12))
 (segment (start 97.5 31) (end 97.9 30.6) (width 0.5) (layer F.Cu) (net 12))
 (segment (start 97.9 30.6) (end 97.9 29.05) (width 0.5) (layer F.Cu) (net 12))
 (segment (start 89 29.05) (end 89 30.5) (width 0.5) (layer F.Cu) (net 12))
 (segment (start 99 30.5) (end 99.5 31) (width 0.5) (layer F.Cu) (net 13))
 (segment (start 99.5 31) (end 107.5 31) (width 0.5) (layer F.Cu) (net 13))
 (segment (start 107.5 31) (end 107.9 30.6) (width 0.5) (layer F.Cu) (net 13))
 (segment (start 107.9 30.6) (end 107.9 29.05) (width 0.5) (layer F.Cu) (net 13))
 (segment (start 99 29.05) (end 99 30.5) (width 0.5) (layer F.Cu) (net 13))
 (segment (start 109 30.5) (end 109.5 31) (width 0.5) (layer F.Cu) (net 14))
 (segment (start 109.5 31) (end 117.5 31) (width 0.5) (layer F.Cu) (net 14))
 (segment (start 117.5 31) (end 117.9 30.6) (width 0.5) (layer F.Cu) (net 14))
 (segment (start 117.9 30.6) (end 117.9 29.05) (width 0.5) (layer F.Cu) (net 14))
 (segment (start 109 29.05) (end 109 30.5) (width 0.5) (layer F.Cu) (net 14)))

